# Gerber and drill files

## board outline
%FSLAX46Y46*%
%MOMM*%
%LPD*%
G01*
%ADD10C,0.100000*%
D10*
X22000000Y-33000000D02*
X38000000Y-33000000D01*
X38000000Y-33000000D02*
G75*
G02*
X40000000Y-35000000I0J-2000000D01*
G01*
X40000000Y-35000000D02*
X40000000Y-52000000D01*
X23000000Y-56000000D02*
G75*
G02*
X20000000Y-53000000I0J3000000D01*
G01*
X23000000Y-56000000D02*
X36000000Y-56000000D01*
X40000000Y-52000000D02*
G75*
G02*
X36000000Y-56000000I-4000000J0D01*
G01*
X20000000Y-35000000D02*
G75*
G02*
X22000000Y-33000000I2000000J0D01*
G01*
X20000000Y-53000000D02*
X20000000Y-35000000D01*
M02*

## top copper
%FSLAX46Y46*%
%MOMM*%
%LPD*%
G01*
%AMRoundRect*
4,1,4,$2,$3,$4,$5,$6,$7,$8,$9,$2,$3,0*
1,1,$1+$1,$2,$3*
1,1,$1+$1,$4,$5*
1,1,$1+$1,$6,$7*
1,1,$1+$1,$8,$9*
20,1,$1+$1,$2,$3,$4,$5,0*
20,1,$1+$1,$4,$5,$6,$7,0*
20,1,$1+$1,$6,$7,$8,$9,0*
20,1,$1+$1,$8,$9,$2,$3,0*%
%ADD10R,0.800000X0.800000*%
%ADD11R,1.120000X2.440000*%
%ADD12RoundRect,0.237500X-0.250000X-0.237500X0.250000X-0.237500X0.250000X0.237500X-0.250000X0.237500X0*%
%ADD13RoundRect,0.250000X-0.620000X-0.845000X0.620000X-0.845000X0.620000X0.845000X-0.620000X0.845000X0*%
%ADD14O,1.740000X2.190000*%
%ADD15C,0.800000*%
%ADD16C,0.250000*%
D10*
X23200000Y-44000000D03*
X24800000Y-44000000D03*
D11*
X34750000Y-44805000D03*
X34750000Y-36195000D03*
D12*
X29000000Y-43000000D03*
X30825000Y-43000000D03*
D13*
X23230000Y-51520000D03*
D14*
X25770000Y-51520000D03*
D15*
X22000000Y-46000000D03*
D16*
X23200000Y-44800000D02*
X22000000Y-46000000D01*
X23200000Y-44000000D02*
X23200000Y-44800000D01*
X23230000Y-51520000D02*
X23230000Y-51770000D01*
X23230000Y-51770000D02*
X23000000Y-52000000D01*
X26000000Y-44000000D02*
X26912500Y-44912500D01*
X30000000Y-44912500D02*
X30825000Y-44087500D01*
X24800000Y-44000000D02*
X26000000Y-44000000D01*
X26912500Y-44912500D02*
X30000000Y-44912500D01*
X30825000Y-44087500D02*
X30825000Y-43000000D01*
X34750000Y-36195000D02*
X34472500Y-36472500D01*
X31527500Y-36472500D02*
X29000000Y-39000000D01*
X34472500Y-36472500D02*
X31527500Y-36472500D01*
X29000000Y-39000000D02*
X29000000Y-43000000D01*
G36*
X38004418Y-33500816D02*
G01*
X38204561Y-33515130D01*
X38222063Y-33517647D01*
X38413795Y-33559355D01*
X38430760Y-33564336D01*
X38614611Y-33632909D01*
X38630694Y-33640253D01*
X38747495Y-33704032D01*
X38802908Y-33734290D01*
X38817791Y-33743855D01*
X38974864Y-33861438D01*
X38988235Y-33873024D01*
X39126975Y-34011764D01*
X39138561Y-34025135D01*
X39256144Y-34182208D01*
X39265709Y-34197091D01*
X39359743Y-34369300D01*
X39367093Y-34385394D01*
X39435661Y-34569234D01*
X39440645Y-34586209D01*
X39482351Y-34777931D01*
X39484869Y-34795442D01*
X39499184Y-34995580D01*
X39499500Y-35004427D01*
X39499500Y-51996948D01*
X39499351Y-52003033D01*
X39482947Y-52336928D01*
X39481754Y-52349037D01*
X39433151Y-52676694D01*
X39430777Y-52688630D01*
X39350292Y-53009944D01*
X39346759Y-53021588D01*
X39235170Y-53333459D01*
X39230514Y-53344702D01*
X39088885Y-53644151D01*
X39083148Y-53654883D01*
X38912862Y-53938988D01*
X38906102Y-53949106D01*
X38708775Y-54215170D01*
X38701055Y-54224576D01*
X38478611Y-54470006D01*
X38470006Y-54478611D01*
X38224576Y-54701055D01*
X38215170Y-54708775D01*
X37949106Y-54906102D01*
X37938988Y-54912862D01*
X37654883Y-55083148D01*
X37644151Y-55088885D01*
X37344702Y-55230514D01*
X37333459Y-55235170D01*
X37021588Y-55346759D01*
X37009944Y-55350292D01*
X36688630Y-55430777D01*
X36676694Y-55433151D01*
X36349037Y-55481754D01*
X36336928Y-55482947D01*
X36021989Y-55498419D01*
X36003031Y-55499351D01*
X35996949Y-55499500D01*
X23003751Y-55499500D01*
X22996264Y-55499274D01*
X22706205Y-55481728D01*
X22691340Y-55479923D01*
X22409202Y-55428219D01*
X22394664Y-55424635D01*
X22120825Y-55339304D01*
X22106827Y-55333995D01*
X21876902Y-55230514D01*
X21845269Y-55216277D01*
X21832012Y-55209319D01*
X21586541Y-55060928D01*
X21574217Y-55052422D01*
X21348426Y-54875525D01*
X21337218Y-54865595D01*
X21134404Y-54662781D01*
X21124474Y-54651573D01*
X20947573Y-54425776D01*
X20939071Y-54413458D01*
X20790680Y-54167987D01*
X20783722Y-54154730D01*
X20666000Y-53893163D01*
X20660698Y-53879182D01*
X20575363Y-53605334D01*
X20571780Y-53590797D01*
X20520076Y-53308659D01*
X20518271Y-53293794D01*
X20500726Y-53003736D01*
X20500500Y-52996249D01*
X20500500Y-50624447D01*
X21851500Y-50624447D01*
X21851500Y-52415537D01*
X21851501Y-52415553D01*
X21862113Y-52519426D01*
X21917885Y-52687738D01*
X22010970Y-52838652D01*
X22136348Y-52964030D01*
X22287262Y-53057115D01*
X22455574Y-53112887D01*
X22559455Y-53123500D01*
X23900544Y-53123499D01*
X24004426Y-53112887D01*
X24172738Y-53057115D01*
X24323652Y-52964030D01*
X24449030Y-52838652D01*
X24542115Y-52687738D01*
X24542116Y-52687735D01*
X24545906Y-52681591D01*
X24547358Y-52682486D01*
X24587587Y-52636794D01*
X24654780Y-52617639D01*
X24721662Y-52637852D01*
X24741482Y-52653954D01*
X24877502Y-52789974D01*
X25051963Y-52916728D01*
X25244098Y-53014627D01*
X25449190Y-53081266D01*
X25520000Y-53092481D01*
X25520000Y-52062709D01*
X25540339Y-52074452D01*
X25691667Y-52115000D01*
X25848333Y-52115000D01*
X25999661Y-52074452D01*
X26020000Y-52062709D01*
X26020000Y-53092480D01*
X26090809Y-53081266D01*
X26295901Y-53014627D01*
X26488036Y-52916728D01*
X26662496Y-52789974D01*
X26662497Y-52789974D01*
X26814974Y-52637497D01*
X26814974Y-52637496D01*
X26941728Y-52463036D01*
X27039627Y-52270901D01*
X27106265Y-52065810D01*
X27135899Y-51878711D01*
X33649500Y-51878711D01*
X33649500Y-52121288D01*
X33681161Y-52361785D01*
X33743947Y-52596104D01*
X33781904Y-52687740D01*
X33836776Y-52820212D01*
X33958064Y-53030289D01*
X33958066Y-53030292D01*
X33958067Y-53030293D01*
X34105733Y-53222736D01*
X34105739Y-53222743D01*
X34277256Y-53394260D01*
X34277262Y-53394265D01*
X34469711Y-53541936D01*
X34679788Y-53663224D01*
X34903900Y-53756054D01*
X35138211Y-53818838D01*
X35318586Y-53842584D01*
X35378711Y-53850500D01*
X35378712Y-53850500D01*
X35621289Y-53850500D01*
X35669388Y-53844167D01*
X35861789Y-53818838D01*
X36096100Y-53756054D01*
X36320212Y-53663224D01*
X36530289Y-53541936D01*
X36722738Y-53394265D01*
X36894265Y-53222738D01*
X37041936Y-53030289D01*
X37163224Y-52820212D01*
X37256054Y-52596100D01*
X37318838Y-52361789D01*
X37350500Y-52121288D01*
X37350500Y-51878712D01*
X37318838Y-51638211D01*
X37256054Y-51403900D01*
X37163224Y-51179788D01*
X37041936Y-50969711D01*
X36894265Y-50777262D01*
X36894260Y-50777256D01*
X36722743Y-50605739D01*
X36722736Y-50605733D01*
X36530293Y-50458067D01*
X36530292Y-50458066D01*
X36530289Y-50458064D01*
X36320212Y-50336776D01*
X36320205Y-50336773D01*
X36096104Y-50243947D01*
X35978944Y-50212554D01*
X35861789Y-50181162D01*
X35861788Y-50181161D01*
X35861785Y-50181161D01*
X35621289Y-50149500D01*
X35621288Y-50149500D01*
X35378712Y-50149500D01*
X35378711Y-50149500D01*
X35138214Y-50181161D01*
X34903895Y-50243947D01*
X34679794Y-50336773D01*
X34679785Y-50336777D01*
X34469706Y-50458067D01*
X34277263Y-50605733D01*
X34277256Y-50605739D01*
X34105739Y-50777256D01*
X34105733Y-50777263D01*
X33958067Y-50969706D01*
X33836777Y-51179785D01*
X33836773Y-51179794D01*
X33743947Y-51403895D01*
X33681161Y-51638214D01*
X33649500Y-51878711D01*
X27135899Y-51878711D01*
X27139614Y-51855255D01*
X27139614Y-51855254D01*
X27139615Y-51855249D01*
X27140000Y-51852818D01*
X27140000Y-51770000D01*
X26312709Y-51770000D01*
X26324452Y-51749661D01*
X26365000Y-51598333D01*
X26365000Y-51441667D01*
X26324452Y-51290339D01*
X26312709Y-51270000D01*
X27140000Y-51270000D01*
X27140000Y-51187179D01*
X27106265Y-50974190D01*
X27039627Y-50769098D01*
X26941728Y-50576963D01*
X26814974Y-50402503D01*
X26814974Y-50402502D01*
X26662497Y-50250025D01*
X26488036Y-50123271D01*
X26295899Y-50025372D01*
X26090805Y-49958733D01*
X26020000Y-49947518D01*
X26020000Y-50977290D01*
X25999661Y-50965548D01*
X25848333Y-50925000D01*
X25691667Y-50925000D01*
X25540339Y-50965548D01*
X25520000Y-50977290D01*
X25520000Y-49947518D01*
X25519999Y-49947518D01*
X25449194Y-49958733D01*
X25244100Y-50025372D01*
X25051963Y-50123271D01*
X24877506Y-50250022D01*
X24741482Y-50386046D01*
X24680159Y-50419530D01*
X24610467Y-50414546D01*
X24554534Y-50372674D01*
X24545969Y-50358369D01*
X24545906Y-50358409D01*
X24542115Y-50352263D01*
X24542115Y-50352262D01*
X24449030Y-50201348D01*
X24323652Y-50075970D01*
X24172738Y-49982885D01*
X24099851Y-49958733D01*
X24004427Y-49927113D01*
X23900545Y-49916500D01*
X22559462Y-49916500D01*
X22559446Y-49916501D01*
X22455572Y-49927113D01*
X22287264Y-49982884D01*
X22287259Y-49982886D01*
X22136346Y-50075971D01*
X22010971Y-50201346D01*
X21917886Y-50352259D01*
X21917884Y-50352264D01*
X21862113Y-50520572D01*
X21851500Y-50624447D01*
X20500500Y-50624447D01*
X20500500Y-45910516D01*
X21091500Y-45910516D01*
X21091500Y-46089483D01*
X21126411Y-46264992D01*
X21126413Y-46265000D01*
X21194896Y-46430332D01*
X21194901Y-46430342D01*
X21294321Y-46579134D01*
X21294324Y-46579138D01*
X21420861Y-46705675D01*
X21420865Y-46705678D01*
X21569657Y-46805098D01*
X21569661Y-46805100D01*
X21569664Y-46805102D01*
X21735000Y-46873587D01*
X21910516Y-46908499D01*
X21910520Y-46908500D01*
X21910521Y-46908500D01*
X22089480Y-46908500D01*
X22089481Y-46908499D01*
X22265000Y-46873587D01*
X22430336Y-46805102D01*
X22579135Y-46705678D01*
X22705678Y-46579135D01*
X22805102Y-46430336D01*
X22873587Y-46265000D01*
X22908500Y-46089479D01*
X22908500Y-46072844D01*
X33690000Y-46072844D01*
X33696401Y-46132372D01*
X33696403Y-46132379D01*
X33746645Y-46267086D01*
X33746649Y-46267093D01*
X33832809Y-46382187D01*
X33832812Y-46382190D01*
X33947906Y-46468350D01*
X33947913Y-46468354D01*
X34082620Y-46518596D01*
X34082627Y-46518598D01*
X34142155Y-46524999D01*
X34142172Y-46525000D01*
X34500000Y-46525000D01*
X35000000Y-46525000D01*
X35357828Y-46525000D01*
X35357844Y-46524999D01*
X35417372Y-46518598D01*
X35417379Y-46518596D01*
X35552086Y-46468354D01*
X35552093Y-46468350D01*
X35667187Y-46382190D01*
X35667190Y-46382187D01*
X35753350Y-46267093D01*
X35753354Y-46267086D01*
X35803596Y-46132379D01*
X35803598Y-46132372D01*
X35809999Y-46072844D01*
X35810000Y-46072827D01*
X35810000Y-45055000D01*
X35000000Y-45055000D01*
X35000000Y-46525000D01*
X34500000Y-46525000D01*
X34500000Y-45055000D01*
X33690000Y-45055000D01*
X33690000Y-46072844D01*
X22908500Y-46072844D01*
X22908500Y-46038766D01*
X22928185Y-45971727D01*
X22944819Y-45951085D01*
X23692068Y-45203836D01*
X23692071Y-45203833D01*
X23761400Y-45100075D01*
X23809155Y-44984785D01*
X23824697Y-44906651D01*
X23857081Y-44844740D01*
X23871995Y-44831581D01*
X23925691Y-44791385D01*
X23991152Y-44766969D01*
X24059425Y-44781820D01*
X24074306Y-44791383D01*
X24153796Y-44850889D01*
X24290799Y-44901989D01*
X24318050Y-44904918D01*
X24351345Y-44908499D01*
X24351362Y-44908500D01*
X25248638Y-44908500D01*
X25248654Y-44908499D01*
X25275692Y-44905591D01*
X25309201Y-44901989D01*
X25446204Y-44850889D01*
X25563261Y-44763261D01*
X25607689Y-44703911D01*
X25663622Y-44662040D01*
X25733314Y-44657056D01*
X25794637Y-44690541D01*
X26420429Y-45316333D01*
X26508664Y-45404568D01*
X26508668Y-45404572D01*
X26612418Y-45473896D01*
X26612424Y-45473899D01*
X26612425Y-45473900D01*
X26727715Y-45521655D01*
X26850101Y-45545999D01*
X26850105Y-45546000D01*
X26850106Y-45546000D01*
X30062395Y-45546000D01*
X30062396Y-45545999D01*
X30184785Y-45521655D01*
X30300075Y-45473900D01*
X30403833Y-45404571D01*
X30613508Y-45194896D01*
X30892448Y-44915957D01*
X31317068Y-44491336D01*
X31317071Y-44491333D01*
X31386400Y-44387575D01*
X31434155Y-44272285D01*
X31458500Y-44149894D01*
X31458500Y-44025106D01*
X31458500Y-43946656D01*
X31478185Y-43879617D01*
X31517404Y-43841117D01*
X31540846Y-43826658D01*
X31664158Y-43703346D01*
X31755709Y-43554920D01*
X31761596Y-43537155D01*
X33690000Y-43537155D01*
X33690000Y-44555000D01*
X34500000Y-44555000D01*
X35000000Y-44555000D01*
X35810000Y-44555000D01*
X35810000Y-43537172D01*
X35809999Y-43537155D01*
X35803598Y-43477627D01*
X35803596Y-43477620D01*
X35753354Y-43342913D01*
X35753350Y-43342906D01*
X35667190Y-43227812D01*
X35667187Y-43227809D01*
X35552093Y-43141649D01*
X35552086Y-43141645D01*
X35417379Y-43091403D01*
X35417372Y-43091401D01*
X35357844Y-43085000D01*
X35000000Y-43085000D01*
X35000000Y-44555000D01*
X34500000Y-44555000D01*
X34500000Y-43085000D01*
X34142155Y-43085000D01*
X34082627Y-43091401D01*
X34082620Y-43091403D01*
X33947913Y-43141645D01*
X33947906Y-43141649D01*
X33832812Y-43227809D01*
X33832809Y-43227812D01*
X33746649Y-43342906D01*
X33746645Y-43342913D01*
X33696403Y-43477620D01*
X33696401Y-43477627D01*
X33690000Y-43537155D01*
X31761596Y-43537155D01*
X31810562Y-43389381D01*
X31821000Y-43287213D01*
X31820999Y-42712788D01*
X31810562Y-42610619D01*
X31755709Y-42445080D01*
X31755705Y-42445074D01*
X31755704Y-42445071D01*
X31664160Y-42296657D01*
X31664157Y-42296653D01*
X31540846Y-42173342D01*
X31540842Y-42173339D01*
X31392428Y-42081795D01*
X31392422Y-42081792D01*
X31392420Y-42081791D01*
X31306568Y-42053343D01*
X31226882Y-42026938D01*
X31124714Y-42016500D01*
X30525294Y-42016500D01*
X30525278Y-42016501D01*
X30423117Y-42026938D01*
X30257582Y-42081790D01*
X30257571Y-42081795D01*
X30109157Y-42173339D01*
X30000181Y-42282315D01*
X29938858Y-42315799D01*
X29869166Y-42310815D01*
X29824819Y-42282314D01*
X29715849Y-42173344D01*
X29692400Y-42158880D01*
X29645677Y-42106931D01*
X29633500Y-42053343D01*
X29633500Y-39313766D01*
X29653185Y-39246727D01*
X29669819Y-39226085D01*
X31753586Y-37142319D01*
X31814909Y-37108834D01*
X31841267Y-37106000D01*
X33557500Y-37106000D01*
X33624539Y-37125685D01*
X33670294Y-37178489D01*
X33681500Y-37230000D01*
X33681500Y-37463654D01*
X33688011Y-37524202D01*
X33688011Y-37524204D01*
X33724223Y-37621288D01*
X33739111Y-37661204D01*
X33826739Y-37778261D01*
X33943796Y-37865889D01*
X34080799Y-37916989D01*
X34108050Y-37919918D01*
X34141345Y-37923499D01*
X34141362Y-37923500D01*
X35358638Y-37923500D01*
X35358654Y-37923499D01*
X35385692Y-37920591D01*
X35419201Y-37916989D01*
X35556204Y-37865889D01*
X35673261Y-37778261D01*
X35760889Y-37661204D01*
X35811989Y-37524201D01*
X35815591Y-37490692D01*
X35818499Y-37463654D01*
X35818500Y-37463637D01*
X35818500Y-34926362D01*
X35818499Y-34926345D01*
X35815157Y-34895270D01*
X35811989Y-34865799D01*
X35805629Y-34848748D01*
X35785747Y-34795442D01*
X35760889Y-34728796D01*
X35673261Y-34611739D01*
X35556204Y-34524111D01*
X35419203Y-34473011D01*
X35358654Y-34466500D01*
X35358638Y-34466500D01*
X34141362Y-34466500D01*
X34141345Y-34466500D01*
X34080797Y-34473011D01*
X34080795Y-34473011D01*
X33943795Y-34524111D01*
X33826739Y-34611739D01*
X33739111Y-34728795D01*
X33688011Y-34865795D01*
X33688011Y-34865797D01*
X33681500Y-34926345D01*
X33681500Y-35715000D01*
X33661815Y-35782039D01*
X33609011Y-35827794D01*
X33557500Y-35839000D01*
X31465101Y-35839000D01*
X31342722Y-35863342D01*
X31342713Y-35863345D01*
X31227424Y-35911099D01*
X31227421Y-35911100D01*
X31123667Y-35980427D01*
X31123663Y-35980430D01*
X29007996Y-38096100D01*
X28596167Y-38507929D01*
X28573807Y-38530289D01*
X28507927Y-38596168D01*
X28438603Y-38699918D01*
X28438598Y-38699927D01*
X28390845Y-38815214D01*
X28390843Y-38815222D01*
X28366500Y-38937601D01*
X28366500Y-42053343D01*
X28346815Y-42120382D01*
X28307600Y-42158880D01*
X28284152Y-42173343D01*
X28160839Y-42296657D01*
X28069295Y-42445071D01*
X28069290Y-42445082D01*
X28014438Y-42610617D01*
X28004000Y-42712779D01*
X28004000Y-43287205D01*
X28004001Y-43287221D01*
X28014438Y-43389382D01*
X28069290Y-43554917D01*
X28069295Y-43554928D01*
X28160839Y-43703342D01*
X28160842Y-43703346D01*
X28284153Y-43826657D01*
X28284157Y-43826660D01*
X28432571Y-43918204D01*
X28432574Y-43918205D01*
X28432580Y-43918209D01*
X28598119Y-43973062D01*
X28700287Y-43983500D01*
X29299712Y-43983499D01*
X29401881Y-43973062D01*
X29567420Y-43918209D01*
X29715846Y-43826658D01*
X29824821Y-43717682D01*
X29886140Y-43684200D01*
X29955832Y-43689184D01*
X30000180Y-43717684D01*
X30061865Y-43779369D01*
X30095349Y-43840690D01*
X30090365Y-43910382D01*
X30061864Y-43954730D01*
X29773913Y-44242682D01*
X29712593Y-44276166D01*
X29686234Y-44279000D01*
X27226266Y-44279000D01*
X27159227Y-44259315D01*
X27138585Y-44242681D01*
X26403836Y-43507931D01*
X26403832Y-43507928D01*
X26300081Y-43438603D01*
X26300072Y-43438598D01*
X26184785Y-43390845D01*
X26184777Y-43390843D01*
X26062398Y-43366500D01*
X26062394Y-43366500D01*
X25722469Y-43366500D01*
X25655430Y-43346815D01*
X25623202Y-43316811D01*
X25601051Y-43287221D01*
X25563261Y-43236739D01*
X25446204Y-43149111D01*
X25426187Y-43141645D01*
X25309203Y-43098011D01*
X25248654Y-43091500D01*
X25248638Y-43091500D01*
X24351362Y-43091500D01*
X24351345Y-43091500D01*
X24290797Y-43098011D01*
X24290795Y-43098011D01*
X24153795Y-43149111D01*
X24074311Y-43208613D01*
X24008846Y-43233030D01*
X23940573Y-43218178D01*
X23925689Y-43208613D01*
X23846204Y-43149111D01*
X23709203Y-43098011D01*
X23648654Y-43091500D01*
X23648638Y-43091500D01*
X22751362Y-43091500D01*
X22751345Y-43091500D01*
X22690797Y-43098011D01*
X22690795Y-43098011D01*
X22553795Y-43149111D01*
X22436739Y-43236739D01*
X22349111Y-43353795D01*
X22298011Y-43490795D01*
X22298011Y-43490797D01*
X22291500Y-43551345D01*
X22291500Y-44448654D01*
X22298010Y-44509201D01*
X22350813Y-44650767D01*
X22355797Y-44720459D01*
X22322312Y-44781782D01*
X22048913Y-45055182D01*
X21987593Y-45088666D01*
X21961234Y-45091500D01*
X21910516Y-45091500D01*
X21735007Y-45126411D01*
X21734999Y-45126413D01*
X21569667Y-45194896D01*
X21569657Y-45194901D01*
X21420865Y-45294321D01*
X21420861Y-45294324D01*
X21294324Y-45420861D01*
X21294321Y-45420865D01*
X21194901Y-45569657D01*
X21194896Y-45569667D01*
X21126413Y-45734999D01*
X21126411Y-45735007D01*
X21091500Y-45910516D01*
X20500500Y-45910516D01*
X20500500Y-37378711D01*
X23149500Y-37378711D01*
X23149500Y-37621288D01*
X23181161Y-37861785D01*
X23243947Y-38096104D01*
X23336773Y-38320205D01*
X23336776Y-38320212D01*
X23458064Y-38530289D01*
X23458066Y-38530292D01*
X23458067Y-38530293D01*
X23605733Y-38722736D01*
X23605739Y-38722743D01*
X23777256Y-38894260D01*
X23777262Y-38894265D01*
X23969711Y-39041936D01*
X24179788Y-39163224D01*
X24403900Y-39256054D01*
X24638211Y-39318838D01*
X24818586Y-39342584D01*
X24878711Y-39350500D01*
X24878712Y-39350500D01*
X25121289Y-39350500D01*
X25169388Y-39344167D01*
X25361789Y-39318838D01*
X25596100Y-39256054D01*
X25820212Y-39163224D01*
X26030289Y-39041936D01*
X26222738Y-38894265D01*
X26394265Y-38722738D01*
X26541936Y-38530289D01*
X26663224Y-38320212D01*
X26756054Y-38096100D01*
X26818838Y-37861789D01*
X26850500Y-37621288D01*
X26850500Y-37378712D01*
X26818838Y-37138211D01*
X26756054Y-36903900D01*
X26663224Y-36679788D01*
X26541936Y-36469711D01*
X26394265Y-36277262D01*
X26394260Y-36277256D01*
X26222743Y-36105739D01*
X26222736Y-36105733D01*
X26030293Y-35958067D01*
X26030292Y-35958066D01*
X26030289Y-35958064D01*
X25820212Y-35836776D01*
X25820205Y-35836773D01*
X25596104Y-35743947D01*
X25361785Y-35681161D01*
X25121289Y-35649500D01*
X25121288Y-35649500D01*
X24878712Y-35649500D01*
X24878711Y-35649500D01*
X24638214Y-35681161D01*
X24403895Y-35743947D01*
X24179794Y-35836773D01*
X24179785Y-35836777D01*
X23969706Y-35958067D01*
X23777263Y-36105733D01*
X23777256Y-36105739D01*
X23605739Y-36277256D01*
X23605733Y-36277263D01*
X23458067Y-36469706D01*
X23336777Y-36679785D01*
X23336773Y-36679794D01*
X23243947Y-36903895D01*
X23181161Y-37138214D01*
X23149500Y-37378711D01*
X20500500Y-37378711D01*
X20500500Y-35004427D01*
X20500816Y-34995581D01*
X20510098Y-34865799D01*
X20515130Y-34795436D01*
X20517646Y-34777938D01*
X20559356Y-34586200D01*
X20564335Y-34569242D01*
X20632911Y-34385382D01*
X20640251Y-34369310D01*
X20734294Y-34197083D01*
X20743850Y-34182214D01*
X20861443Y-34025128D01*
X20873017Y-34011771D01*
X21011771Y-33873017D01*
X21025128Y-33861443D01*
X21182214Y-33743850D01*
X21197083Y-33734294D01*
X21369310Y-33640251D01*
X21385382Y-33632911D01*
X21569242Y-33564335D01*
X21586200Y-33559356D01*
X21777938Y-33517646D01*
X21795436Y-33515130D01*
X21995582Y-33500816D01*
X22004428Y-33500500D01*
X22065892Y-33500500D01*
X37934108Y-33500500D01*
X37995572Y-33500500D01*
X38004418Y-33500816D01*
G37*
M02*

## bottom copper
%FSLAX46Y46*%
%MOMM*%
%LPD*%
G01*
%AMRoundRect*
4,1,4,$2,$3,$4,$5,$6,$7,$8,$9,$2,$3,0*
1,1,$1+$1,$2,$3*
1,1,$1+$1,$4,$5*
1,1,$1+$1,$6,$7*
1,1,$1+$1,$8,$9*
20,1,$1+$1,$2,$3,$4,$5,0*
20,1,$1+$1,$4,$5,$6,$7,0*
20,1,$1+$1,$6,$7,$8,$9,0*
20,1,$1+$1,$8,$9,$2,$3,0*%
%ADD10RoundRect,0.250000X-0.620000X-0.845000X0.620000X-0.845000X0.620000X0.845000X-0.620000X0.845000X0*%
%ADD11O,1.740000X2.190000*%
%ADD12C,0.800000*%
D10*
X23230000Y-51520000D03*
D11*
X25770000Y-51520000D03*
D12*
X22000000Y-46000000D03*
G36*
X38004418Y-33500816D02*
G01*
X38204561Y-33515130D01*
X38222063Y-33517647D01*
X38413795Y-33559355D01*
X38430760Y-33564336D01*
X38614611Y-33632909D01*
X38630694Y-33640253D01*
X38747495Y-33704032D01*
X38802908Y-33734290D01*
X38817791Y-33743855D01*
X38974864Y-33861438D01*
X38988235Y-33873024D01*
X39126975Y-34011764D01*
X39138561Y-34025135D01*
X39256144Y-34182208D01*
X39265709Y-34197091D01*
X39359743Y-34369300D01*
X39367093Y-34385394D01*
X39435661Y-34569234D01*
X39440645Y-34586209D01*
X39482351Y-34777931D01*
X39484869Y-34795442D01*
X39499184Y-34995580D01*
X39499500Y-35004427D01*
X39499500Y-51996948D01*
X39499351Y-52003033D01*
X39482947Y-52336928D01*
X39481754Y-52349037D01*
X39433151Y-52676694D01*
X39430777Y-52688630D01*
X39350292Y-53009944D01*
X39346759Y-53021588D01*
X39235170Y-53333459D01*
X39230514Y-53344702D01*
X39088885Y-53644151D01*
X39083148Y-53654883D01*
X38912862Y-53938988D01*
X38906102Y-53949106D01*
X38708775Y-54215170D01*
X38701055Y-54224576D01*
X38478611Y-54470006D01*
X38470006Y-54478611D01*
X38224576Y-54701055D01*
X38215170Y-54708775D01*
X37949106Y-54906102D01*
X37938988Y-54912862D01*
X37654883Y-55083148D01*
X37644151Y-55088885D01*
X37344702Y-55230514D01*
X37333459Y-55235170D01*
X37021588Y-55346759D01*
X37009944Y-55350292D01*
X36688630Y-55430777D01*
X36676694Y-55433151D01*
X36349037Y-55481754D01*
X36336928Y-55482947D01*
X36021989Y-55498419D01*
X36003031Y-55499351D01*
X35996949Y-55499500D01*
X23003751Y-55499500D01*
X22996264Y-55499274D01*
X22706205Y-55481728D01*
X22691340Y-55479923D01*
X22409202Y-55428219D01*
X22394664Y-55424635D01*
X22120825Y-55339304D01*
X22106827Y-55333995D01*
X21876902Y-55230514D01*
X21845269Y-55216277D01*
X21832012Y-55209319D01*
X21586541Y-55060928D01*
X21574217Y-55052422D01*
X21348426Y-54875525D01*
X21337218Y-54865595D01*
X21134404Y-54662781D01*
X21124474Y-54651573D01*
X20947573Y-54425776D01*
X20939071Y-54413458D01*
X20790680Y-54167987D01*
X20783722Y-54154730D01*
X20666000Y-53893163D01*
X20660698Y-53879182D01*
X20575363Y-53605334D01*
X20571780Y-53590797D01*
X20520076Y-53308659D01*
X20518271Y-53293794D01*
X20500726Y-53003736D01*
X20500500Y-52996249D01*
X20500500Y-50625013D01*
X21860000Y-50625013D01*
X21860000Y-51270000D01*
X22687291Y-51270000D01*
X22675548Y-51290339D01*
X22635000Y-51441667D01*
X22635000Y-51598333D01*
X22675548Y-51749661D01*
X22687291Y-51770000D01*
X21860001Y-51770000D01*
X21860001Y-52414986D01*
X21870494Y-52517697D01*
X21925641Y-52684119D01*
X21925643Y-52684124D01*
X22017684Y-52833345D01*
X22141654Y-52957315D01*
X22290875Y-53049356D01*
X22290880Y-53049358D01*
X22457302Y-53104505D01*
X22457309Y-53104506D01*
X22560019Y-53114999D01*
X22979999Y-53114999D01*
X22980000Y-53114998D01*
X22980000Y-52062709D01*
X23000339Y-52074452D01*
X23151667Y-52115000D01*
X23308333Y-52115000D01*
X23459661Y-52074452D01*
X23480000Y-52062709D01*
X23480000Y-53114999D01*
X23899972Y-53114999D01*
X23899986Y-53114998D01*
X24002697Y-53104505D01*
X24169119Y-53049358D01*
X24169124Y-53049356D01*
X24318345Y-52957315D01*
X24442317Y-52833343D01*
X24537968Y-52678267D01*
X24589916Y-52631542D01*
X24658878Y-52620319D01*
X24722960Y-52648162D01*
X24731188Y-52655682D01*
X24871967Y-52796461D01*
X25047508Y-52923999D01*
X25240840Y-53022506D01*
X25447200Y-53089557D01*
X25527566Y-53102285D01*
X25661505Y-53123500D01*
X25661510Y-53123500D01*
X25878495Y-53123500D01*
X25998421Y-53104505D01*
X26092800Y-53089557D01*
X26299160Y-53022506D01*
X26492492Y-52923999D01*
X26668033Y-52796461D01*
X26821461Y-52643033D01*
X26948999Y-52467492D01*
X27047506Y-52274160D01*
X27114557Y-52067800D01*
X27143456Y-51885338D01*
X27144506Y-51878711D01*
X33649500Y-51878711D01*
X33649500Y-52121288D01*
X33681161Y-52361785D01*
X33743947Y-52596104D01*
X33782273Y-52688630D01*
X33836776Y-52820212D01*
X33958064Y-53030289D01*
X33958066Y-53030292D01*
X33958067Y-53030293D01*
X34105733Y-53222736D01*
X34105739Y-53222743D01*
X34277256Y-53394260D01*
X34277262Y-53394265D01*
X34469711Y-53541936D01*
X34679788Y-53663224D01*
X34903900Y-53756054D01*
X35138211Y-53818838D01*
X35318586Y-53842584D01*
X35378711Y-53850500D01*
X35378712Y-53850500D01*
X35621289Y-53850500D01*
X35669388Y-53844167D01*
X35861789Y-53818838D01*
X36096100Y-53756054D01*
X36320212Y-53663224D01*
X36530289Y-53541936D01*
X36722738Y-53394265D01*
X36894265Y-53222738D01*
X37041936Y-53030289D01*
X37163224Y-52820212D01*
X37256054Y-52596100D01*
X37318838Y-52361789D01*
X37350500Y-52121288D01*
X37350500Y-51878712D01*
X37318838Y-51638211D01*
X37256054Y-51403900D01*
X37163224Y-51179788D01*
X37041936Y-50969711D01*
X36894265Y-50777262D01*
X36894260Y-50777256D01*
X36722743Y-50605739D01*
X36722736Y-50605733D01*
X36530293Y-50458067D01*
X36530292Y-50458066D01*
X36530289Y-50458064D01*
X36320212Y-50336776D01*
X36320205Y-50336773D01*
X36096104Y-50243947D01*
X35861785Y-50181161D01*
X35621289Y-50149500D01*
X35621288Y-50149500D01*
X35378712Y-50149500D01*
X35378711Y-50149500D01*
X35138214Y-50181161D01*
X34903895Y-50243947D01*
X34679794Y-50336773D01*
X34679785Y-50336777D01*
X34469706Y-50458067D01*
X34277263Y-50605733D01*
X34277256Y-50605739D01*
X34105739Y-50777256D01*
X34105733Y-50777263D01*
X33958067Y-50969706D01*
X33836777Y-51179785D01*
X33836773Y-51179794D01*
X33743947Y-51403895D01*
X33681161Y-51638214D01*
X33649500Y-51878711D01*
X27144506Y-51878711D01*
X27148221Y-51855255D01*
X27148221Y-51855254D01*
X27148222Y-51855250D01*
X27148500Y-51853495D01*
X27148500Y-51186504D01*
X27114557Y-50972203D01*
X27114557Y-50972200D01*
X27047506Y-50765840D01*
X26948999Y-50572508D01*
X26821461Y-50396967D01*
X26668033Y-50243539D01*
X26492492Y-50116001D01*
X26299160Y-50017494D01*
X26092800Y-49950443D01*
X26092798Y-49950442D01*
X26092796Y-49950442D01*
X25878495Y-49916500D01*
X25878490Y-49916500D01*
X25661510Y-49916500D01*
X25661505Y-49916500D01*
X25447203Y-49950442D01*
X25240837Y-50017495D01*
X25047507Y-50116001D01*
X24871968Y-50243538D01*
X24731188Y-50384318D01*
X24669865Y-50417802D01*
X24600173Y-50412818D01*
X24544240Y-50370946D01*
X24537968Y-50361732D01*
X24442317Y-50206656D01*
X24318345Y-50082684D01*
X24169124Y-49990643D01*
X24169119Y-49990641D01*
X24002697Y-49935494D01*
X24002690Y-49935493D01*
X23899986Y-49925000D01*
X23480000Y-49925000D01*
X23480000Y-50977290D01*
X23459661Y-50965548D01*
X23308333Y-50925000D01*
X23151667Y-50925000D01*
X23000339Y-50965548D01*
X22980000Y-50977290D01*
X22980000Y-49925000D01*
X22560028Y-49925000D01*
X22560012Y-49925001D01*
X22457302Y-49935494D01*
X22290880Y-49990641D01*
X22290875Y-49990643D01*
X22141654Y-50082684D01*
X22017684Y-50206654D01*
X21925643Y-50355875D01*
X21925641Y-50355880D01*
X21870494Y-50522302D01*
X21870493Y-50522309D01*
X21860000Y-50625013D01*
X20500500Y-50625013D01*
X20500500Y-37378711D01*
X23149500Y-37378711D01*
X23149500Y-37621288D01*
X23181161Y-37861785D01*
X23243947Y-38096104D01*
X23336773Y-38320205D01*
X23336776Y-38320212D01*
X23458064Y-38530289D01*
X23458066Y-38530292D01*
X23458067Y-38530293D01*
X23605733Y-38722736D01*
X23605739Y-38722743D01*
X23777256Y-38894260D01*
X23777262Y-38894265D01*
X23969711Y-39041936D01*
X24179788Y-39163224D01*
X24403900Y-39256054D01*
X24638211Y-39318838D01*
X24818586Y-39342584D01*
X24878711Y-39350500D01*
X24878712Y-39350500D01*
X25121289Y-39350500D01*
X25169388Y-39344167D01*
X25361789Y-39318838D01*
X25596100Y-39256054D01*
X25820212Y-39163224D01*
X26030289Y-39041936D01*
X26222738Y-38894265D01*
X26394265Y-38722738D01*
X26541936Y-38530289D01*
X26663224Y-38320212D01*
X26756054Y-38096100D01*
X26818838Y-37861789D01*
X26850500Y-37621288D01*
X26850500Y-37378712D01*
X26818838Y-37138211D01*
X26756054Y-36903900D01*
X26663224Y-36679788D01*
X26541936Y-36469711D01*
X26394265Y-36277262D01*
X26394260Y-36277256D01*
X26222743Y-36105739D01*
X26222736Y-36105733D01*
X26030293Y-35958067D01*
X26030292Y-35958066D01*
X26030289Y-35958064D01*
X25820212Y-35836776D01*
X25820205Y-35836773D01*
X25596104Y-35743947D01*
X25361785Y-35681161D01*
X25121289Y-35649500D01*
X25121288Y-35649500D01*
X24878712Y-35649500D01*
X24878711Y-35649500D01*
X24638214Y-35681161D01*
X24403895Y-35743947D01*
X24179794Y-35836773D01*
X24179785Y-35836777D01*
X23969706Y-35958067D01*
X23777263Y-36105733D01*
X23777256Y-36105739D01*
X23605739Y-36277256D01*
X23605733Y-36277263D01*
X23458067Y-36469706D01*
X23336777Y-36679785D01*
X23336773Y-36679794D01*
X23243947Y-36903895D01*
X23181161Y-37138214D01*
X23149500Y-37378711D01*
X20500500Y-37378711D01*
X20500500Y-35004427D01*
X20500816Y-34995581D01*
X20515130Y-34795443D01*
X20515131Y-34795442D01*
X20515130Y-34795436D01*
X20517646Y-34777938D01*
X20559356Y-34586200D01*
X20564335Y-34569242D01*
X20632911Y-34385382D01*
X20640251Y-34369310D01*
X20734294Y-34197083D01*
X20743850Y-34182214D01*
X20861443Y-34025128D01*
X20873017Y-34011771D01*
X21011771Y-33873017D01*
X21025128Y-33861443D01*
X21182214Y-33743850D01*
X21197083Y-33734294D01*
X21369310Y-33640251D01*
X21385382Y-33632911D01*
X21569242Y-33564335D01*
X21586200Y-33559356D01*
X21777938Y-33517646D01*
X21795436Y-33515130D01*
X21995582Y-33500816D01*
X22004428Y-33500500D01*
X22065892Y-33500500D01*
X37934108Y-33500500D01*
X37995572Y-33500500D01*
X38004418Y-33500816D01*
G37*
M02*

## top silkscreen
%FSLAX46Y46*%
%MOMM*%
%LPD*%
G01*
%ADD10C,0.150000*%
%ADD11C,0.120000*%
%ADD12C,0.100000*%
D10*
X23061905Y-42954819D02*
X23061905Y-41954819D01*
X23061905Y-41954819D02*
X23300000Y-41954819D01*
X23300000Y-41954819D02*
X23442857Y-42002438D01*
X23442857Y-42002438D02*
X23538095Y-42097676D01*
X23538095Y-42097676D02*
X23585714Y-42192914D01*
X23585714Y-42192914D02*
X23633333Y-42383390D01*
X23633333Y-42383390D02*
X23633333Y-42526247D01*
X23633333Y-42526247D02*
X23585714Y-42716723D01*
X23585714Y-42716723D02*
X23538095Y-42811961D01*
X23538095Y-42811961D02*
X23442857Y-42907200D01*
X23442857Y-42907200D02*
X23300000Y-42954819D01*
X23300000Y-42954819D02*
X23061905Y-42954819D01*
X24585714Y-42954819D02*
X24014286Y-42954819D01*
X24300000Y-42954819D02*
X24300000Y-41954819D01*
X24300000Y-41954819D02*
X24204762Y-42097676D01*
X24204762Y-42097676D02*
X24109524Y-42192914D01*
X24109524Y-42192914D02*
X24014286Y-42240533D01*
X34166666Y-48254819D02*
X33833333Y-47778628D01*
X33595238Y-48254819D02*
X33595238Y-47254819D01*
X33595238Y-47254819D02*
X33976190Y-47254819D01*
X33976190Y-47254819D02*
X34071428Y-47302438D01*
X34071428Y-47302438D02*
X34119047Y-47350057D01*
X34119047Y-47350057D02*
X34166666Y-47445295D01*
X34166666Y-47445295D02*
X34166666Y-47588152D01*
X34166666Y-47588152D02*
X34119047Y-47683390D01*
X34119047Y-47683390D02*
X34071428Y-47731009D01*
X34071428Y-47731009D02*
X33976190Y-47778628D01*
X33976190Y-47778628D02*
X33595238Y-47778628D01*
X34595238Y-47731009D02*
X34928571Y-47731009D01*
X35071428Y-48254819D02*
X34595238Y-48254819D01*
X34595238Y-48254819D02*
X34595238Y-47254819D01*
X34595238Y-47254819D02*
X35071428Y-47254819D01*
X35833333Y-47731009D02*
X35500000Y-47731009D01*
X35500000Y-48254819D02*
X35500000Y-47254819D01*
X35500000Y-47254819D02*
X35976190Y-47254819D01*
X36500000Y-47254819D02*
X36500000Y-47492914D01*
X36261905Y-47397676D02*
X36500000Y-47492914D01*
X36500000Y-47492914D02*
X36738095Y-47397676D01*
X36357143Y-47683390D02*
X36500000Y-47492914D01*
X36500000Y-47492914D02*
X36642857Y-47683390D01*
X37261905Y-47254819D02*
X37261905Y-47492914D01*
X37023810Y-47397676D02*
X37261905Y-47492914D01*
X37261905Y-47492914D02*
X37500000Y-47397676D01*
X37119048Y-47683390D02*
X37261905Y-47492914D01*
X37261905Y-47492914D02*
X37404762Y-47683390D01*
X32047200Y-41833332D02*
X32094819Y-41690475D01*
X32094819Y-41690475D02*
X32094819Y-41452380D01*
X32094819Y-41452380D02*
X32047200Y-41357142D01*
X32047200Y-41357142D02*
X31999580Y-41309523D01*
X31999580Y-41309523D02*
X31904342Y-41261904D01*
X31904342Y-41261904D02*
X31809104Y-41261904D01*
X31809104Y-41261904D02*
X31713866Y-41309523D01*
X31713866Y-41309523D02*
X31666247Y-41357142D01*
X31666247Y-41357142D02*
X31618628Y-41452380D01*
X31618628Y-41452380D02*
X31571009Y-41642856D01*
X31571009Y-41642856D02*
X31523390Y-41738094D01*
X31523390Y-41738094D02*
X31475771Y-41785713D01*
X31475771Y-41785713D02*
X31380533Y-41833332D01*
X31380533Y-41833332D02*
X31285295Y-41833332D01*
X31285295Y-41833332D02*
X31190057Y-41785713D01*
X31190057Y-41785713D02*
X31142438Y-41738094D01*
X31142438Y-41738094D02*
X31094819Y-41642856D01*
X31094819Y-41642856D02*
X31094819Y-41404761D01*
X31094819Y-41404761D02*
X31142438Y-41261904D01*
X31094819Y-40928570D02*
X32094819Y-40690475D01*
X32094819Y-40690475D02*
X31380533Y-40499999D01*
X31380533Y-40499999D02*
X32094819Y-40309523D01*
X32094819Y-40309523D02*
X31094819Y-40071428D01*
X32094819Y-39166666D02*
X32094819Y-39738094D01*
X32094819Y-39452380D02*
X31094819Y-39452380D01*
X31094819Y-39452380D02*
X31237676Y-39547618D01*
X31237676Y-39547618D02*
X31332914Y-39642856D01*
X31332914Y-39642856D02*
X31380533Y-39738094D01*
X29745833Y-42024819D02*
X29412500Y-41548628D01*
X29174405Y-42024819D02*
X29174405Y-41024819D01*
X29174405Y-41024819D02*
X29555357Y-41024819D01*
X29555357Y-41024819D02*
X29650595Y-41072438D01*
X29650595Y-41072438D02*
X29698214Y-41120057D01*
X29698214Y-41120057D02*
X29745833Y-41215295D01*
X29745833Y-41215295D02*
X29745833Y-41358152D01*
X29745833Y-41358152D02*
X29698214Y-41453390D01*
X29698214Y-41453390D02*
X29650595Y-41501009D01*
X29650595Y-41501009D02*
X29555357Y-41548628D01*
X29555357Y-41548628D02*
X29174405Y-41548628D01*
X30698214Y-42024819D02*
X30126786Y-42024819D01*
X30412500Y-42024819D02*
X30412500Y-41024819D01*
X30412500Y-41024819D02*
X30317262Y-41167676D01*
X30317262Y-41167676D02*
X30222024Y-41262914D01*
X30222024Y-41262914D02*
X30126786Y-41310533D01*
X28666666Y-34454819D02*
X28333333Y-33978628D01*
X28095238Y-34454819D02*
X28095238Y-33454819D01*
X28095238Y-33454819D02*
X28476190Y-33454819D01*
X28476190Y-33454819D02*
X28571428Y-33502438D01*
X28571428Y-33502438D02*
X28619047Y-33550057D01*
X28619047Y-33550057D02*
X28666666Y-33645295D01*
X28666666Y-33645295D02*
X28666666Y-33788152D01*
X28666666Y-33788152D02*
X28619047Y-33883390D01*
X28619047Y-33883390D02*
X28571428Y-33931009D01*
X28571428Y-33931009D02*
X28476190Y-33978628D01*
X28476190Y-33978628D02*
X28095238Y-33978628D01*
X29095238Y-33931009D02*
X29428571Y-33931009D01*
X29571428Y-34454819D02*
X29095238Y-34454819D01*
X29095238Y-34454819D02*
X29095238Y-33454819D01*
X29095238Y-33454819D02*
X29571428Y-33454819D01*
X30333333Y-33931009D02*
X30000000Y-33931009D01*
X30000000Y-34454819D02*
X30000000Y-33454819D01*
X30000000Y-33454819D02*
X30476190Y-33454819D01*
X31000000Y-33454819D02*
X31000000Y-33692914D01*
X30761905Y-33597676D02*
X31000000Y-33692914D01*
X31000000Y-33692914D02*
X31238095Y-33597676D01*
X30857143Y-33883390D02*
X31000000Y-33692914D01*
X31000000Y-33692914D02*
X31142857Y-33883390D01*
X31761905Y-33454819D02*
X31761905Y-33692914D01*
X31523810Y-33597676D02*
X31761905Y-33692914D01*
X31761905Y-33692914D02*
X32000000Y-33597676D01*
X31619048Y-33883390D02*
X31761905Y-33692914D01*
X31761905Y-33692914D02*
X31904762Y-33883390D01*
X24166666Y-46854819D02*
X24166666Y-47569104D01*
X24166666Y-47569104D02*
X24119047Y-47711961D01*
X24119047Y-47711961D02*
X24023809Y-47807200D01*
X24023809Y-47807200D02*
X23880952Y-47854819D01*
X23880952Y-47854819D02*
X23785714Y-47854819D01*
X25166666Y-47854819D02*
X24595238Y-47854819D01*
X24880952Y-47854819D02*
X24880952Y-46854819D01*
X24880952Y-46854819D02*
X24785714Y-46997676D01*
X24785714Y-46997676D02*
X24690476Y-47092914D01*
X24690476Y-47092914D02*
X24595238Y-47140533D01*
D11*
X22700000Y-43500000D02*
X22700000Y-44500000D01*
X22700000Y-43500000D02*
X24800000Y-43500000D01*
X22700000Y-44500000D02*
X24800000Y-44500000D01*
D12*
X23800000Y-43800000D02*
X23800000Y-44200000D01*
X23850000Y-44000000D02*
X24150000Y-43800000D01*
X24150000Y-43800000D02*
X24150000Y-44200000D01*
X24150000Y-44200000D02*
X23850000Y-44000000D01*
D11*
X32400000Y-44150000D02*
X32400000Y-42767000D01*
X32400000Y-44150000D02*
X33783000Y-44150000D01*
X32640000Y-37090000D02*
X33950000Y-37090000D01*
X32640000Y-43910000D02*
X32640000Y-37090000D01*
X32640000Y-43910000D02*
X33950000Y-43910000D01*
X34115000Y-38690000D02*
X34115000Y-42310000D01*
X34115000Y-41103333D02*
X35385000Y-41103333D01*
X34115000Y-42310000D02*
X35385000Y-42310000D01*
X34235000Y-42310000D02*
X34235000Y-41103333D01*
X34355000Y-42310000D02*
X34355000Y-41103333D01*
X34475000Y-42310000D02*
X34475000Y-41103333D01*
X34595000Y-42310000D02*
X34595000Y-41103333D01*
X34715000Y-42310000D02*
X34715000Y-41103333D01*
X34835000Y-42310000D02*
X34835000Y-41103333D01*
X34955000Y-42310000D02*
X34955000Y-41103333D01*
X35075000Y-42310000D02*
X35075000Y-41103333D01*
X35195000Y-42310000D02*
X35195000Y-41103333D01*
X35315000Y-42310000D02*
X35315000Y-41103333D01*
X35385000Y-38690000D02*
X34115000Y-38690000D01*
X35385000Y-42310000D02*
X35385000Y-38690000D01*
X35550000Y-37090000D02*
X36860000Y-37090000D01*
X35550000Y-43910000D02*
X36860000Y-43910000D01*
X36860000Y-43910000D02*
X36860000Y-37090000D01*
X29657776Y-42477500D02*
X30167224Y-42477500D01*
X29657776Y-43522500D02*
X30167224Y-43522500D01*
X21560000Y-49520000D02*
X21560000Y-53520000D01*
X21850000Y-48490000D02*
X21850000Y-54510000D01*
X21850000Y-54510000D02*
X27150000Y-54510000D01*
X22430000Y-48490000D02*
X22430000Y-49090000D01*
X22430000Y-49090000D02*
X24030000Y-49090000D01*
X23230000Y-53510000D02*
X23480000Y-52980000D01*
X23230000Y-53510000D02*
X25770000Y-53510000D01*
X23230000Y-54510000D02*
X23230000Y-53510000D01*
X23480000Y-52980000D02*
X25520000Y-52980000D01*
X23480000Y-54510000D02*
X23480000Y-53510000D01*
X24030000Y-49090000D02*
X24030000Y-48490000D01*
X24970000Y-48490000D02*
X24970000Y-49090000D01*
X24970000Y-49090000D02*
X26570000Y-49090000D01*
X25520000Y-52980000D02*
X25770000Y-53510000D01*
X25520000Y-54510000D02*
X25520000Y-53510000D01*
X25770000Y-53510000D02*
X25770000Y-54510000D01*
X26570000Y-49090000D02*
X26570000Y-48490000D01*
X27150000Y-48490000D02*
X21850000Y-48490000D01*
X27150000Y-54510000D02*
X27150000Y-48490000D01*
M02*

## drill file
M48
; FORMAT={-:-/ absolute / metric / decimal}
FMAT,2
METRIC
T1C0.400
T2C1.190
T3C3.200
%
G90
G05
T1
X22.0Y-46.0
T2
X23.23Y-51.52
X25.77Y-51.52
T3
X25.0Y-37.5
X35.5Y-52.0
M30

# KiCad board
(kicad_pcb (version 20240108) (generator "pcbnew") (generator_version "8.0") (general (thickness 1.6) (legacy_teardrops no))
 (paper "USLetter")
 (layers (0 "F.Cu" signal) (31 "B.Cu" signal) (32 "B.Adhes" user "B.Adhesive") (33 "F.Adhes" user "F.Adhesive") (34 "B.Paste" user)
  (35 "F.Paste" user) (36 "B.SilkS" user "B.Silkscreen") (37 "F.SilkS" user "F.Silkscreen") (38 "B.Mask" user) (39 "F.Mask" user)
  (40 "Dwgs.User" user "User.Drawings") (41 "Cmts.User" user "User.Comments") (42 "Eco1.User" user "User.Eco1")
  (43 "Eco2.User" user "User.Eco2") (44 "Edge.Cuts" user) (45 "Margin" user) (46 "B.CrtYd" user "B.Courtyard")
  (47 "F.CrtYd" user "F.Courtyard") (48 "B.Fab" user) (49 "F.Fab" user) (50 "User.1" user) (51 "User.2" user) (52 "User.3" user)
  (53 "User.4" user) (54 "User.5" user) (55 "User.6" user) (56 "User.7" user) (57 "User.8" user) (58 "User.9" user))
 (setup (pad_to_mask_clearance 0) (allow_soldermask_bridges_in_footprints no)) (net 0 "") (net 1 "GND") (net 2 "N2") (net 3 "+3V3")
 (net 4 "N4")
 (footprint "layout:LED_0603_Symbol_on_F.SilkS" (layer "F.Cu") (at 24 44)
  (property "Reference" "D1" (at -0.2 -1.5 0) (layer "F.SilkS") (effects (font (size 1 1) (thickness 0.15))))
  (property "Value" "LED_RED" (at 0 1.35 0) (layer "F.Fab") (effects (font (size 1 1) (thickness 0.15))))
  (fp_line (start -1.3 -0.5) (end -1.3 0.5) (stroke (width 0.12) (type solid)) (layer "F.SilkS"))
  (fp_line (start -1.3 -0.5) (end 0.8 -0.5) (stroke (width 0.12) (type solid)) (layer "F.SilkS"))
  (fp_line (start -1.3 0.5) (end 0.8 0.5) (stroke (width 0.12) (type solid)) (layer "F.SilkS"))
  (fp_line (start -0.2 -0.2) (end -0.2 0.2) (stroke (width 0.1) (type solid)) (layer "F.SilkS"))
  (fp_line (start -0.15 0) (end 0.15 -0.2) (stroke (width 0.1) (type solid)) (layer "F.SilkS"))
  (fp_line (start 0.15 -0.2) (end 0.15 0.2) (stroke (width 0.1) (type solid)) (layer "F.SilkS"))
  (fp_line (start 0.15 0.2) (end -0.15 0) (stroke (width 0.1) (type solid)) (layer "F.SilkS"))
  (pad "1" smd rect (at -0.8 0 180) (size 0.8 0.8) (layers "F.Cu" "F.Paste" "F.Mask") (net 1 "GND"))
  (pad "2" smd rect (at 0.8 0 180) (size 0.8 0.8) (layers "F.Cu" "F.Paste" "F.Mask") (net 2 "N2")))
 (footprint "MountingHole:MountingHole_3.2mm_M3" (layer "F.Cu") (at 35.5 52)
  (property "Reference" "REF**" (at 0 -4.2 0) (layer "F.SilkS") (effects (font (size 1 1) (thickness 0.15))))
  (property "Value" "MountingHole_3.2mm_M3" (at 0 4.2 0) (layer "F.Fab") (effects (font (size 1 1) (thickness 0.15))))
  (pad "" np_thru_hole circle (at 0 0) (size 3.2 3.2) (drill 3.2) (layers "*.Cu" "*.Mask")))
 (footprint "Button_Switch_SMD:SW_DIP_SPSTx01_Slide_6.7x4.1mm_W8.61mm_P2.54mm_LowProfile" (layer "F.Cu") (at 34.75 40.5 90)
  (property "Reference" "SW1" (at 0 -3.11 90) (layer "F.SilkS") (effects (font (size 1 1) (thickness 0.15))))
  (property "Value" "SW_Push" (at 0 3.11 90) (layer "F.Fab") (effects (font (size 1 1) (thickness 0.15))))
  (fp_line (start -3.65 -2.35) (end -2.267 -2.35) (stroke (width 0.12) (type solid)) (layer "F.SilkS"))
  (fp_line (start -3.65 -2.35) (end -3.65 -0.967) (stroke (width 0.12) (type solid)) (layer "F.SilkS"))
  (fp_line (start 3.41 -2.11) (end 3.41 -0.8) (stroke (width 0.12) (type solid)) (layer "F.SilkS"))
  (fp_line (start -3.41 -2.11) (end 3.41 -2.11) (stroke (width 0.12) (type solid)) (layer "F.SilkS"))
  (fp_line (start -3.41 -2.11) (end -3.41 -0.8) (stroke (width 0.12) (type solid)) (layer "F.SilkS"))
  (fp_line (start 1.81 -0.635) (end -1.81 -0.635) (stroke (width 0.12) (type solid)) (layer "F.SilkS"))
  (fp_line (start -0.603333 -0.635) (end -0.603333 0.635) (stroke (width 0.12) (type solid)) (layer "F.SilkS"))
  (fp_line (start -1.81 -0.635) (end -1.81 0.635) (stroke (width 0.12) (type solid)) (layer "F.SilkS"))
  (fp_line (start -1.81 -0.515) (end -0.603333 -0.515) (stroke (width 0.12) (type solid)) (layer "F.SilkS"))
  (fp_line (start -1.81 -0.395) (end -0.603333 -0.395) (stroke (width 0.12) (type solid)) (layer "F.SilkS"))
  (fp_line (start -1.81 -0.275) (end -0.603333 -0.275) (stroke (width 0.12) (type solid)) (layer "F.SilkS"))
  (fp_line (start -1.81 -0.155) (end -0.603333 -0.155) (stroke (width 0.12) (type solid)) (layer "F.SilkS"))
  (fp_line (start -1.81 -0.035) (end -0.603333 -0.035) (stroke (width 0.12) (type solid)) (layer "F.SilkS"))
  (fp_line (start -1.81 0.085) (end -0.603333 0.085) (stroke (width 0.12) (type solid)) (layer "F.SilkS"))
  (fp_line (start -1.81 0.205) (end -0.603333 0.205) (stroke (width 0.12) (type solid)) (layer "F.SilkS"))
  (fp_line (start -1.81 0.325) (end -0.603333 0.325) (stroke (width 0.12) (type solid)) (layer "F.SilkS"))
  (fp_line (start -1.81 0.445) (end -0.603333 0.445) (stroke (width 0.12) (type solid)) (layer "F.SilkS"))
  (fp_line (start -1.81 0.565) (end -0.603333 0.565) (stroke (width 0.12) (type solid)) (layer "F.SilkS"))
  (fp_line (start 1.81 0.635) (end 1.81 -0.635) (stroke (width 0.12) (type solid)) (layer "F.SilkS"))
  (fp_line (start -1.81 0.635) (end 1.81 0.635) (stroke (width 0.12) (type solid)) (layer "F.SilkS"))
  (fp_line (start 3.41 0.8) (end 3.41 2.11) (stroke (width 0.12) (type solid)) (layer "F.SilkS"))
  (fp_line (start -3.41 0.8) (end -3.41 2.11) (stroke (width 0.12) (type solid)) (layer "F.SilkS"))
  (fp_line (start -3.41 2.11) (end 3.41 2.11) (stroke (width 0.12) (type solid)) (layer "F.SilkS"))
  (pad "1" smd rect (at -4.305 0 90) (size 2.44 1.12) (layers "F.Cu" "F.Paste" "F.Mask") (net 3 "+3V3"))
  (pad "2" smd rect (at 4.305 0 90) (size 2.44 1.12) (layers "F.Cu" "F.Paste" "F.Mask") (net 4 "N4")))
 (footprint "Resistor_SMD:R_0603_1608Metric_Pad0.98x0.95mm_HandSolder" (layer "F.Cu") (at 29.9125 43)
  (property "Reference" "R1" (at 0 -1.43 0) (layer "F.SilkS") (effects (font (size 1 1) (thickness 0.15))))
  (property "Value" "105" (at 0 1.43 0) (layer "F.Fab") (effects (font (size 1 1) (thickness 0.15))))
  (fp_line (start -0.254724 -0.5225) (end 0.254724 -0.5225) (stroke (width 0.12) (type solid)) (layer "F.SilkS"))
  (fp_line (start -0.254724 0.5225) (end 0.254724 0.5225) (stroke (width 0.12) (type solid)) (layer "F.SilkS"))
  (pad "1" smd roundrect (at -0.9125 0) (size 0.975 0.95) (layers "F.Cu" "F.Paste" "F.Mask") (roundrect_rratio 0.25) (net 4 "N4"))
  (pad "2" smd roundrect (at 0.9125 0) (size 0.975 0.95) (layers "F.Cu" "F.Paste" "F.Mask") (roundrect_rratio 0.25) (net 2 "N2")))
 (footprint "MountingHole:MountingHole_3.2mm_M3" (layer "F.Cu") (at 25 37.5)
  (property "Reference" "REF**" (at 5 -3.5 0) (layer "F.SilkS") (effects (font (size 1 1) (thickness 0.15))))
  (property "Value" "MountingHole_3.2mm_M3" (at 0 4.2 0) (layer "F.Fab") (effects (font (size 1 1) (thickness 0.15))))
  (pad "" np_thru_hole circle (at 0 0) (size 3.2 3.2) (drill 3.2) (layers "*.Cu" "*.Mask")))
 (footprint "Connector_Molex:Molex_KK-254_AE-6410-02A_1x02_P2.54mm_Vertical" (layer "F.Cu") (at 23.23 51.52)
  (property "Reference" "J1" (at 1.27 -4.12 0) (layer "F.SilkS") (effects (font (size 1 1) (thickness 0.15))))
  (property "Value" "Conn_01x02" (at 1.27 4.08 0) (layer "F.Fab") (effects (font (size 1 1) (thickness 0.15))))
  (fp_line (start -1.67 -2) (end -1.67 2) (stroke (width 0.12) (type solid)) (layer "F.SilkS"))
  (fp_line (start -1.38 -3.03) (end -1.38 2.99) (stroke (width 0.12) (type solid)) (layer "F.SilkS"))
  (fp_line (start -1.38 2.99) (end 3.92 2.99) (stroke (width 0.12) (type solid)) (layer "F.SilkS"))
  (fp_line (start -0.8 -3.03) (end -0.8 -2.43) (stroke (width 0.12) (type solid)) (layer "F.SilkS"))
  (fp_line (start -0.8 -2.43) (end 0.8 -2.43) (stroke (width 0.12) (type solid)) (layer "F.SilkS"))
  (fp_line (start 0 1.99) (end 0.25 1.46) (stroke (width 0.12) (type solid)) (layer "F.SilkS"))
  (fp_line (start 0 1.99) (end 2.54 1.99) (stroke (width 0.12) (type solid)) (layer "F.SilkS"))
  (fp_line (start 0 2.99) (end 0 1.99) (stroke (width 0.12) (type solid)) (layer "F.SilkS"))
  (fp_line (start 0.25 1.46) (end 2.29 1.46) (stroke (width 0.12) (type solid)) (layer "F.SilkS"))
  (fp_line (start 0.25 2.99) (end 0.25 1.99) (stroke (width 0.12) (type solid)) (layer "F.SilkS"))
  (fp_line (start 0.8 -2.43) (end 0.8 -3.03) (stroke (width 0.12) (type solid)) (layer "F.SilkS"))
  (fp_line (start 1.74 -3.03) (end 1.74 -2.43) (stroke (width 0.12) (type solid)) (layer "F.SilkS"))
  (fp_line (start 1.74 -2.43) (end 3.34 -2.43) (stroke (width 0.12) (type solid)) (layer "F.SilkS"))
  (fp_line (start 2.29 1.46) (end 2.54 1.99) (stroke (width 0.12) (type solid)) (layer "F.SilkS"))
  (fp_line (start 2.29 2.99) (end 2.29 1.99) (stroke (width 0.12) (type solid)) (layer "F.SilkS"))
  (fp_line (start 2.54 1.99) (end 2.54 2.99) (stroke (width 0.12) (type solid)) (layer "F.SilkS"))
  (fp_line (start 3.34 -2.43) (end 3.34 -3.03) (stroke (width 0.12) (type solid)) (layer "F.SilkS"))
  (fp_line (start 3.92 -3.03) (end -1.38 -3.03) (stroke (width 0.12) (type solid)) (layer "F.SilkS"))
  (fp_line (start 3.92 2.99) (end 3.92 -3.03) (stroke (width 0.12) (type solid)) (layer "F.SilkS"))
  (pad "1" thru_hole roundrect (at 0 0) (size 1.74 2.19) (drill 1.19) (layers "*.Cu" "*.Mask") (remove_unused_layers no)
   (roundrect_rratio 0.143678) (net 1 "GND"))
  (pad "2" thru_hole oval (at 2.54 0) (size 1.74 2.19) (drill 1.19) (layers "*.Cu" "*.Mask") (remove_unused_layers no) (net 3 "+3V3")))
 (gr_line (start 22 33) (end 38 33) (stroke (width 0.1) (type default)) (layer "Edge.Cuts"))
 (gr_arc (start 38 33) (mid 39.414214 33.585786) (end 40 35) (stroke (width 0.1) (type default)) (layer "Edge.Cuts"))
 (gr_line (start 40 35) (end 40 52) (stroke (width 0.1) (type default)) (layer "Edge.Cuts"))
 (gr_arc (start 23 56) (mid 20.87868 55.12132) (end 20 53) (stroke (width 0.1) (type default)) (layer "Edge.Cuts"))
 (gr_line (start 23 56) (end 36 56) (stroke (width 0.1) (type default)) (layer "Edge.Cuts"))
 (gr_arc (start 40 52) (mid 38.828427 54.828427) (end 36 56) (stroke (width 0.1) (type default)) (layer "Edge.Cuts"))
 (gr_arc (start 20 35) (mid 20.585786 33.585786) (end 22 33) (stroke (width 0.1) (type default)) (layer "Edge.Cuts"))
 (gr_line (start 20 53) (end 20 35) (stroke (width 0.1) (type default)) (layer "Edge.Cuts"))
 (segment (start 23.2 44.8) (end 22 46) (width 0.25) (layer "F.Cu") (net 1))
 (segment (start 23.2 44) (end 23.2 44.8) (width 0.25) (layer "F.Cu") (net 1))
 (segment (start 23.23 51.52) (end 23.23 51.77) (width 0.25) (layer "F.Cu") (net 1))
 (segment (start 23.23 51.77) (end 23 52) (width 0.25) (layer "F.Cu") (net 1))
 (via (at 22 46) (size 0.8) (drill 0.4) (layers "F.Cu" "B.Cu") (free yes) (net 1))
 (segment (start 26 44) (end 26.9125 44.9125) (width 0.25) (layer "F.Cu") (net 2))
 (segment (start 30 44.9125) (end 30.825 44.0875) (width 0.25) (layer "F.Cu") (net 2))
 (segment (start 24.8 44) (end 26 44) (width 0.25) (layer "F.Cu") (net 2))
 (segment (start 26.9125 44.9125) (end 30 44.9125) (width 0.25) (layer "F.Cu") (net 2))
 (segment (start 30.825 44.0875) (end 30.825 43) (width 0.25) (layer "F.Cu") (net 2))
 (segment (start 34.75 36.195) (end 34.4725 36.4725) (width 0.25) (layer "F.Cu") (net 4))
 (segment (start 31.5275 36.4725) (end 29 39) (width 0.25) (layer "F.Cu") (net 4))
 (segment (start 34.4725 36.4725) (end 31.5275 36.4725) (width 0.25) (layer "F.Cu") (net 4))
 (segment (start 29 39) (end 29 43) (width 0.25) (layer "F.Cu") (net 4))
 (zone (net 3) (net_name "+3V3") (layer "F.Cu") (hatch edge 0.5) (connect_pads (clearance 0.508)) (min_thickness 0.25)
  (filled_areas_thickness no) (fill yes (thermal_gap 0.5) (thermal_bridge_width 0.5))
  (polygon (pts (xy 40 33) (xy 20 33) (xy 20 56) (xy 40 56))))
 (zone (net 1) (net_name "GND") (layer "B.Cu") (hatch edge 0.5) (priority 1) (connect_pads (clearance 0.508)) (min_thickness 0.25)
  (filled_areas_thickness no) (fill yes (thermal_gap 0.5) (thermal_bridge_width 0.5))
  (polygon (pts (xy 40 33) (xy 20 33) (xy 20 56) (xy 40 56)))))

